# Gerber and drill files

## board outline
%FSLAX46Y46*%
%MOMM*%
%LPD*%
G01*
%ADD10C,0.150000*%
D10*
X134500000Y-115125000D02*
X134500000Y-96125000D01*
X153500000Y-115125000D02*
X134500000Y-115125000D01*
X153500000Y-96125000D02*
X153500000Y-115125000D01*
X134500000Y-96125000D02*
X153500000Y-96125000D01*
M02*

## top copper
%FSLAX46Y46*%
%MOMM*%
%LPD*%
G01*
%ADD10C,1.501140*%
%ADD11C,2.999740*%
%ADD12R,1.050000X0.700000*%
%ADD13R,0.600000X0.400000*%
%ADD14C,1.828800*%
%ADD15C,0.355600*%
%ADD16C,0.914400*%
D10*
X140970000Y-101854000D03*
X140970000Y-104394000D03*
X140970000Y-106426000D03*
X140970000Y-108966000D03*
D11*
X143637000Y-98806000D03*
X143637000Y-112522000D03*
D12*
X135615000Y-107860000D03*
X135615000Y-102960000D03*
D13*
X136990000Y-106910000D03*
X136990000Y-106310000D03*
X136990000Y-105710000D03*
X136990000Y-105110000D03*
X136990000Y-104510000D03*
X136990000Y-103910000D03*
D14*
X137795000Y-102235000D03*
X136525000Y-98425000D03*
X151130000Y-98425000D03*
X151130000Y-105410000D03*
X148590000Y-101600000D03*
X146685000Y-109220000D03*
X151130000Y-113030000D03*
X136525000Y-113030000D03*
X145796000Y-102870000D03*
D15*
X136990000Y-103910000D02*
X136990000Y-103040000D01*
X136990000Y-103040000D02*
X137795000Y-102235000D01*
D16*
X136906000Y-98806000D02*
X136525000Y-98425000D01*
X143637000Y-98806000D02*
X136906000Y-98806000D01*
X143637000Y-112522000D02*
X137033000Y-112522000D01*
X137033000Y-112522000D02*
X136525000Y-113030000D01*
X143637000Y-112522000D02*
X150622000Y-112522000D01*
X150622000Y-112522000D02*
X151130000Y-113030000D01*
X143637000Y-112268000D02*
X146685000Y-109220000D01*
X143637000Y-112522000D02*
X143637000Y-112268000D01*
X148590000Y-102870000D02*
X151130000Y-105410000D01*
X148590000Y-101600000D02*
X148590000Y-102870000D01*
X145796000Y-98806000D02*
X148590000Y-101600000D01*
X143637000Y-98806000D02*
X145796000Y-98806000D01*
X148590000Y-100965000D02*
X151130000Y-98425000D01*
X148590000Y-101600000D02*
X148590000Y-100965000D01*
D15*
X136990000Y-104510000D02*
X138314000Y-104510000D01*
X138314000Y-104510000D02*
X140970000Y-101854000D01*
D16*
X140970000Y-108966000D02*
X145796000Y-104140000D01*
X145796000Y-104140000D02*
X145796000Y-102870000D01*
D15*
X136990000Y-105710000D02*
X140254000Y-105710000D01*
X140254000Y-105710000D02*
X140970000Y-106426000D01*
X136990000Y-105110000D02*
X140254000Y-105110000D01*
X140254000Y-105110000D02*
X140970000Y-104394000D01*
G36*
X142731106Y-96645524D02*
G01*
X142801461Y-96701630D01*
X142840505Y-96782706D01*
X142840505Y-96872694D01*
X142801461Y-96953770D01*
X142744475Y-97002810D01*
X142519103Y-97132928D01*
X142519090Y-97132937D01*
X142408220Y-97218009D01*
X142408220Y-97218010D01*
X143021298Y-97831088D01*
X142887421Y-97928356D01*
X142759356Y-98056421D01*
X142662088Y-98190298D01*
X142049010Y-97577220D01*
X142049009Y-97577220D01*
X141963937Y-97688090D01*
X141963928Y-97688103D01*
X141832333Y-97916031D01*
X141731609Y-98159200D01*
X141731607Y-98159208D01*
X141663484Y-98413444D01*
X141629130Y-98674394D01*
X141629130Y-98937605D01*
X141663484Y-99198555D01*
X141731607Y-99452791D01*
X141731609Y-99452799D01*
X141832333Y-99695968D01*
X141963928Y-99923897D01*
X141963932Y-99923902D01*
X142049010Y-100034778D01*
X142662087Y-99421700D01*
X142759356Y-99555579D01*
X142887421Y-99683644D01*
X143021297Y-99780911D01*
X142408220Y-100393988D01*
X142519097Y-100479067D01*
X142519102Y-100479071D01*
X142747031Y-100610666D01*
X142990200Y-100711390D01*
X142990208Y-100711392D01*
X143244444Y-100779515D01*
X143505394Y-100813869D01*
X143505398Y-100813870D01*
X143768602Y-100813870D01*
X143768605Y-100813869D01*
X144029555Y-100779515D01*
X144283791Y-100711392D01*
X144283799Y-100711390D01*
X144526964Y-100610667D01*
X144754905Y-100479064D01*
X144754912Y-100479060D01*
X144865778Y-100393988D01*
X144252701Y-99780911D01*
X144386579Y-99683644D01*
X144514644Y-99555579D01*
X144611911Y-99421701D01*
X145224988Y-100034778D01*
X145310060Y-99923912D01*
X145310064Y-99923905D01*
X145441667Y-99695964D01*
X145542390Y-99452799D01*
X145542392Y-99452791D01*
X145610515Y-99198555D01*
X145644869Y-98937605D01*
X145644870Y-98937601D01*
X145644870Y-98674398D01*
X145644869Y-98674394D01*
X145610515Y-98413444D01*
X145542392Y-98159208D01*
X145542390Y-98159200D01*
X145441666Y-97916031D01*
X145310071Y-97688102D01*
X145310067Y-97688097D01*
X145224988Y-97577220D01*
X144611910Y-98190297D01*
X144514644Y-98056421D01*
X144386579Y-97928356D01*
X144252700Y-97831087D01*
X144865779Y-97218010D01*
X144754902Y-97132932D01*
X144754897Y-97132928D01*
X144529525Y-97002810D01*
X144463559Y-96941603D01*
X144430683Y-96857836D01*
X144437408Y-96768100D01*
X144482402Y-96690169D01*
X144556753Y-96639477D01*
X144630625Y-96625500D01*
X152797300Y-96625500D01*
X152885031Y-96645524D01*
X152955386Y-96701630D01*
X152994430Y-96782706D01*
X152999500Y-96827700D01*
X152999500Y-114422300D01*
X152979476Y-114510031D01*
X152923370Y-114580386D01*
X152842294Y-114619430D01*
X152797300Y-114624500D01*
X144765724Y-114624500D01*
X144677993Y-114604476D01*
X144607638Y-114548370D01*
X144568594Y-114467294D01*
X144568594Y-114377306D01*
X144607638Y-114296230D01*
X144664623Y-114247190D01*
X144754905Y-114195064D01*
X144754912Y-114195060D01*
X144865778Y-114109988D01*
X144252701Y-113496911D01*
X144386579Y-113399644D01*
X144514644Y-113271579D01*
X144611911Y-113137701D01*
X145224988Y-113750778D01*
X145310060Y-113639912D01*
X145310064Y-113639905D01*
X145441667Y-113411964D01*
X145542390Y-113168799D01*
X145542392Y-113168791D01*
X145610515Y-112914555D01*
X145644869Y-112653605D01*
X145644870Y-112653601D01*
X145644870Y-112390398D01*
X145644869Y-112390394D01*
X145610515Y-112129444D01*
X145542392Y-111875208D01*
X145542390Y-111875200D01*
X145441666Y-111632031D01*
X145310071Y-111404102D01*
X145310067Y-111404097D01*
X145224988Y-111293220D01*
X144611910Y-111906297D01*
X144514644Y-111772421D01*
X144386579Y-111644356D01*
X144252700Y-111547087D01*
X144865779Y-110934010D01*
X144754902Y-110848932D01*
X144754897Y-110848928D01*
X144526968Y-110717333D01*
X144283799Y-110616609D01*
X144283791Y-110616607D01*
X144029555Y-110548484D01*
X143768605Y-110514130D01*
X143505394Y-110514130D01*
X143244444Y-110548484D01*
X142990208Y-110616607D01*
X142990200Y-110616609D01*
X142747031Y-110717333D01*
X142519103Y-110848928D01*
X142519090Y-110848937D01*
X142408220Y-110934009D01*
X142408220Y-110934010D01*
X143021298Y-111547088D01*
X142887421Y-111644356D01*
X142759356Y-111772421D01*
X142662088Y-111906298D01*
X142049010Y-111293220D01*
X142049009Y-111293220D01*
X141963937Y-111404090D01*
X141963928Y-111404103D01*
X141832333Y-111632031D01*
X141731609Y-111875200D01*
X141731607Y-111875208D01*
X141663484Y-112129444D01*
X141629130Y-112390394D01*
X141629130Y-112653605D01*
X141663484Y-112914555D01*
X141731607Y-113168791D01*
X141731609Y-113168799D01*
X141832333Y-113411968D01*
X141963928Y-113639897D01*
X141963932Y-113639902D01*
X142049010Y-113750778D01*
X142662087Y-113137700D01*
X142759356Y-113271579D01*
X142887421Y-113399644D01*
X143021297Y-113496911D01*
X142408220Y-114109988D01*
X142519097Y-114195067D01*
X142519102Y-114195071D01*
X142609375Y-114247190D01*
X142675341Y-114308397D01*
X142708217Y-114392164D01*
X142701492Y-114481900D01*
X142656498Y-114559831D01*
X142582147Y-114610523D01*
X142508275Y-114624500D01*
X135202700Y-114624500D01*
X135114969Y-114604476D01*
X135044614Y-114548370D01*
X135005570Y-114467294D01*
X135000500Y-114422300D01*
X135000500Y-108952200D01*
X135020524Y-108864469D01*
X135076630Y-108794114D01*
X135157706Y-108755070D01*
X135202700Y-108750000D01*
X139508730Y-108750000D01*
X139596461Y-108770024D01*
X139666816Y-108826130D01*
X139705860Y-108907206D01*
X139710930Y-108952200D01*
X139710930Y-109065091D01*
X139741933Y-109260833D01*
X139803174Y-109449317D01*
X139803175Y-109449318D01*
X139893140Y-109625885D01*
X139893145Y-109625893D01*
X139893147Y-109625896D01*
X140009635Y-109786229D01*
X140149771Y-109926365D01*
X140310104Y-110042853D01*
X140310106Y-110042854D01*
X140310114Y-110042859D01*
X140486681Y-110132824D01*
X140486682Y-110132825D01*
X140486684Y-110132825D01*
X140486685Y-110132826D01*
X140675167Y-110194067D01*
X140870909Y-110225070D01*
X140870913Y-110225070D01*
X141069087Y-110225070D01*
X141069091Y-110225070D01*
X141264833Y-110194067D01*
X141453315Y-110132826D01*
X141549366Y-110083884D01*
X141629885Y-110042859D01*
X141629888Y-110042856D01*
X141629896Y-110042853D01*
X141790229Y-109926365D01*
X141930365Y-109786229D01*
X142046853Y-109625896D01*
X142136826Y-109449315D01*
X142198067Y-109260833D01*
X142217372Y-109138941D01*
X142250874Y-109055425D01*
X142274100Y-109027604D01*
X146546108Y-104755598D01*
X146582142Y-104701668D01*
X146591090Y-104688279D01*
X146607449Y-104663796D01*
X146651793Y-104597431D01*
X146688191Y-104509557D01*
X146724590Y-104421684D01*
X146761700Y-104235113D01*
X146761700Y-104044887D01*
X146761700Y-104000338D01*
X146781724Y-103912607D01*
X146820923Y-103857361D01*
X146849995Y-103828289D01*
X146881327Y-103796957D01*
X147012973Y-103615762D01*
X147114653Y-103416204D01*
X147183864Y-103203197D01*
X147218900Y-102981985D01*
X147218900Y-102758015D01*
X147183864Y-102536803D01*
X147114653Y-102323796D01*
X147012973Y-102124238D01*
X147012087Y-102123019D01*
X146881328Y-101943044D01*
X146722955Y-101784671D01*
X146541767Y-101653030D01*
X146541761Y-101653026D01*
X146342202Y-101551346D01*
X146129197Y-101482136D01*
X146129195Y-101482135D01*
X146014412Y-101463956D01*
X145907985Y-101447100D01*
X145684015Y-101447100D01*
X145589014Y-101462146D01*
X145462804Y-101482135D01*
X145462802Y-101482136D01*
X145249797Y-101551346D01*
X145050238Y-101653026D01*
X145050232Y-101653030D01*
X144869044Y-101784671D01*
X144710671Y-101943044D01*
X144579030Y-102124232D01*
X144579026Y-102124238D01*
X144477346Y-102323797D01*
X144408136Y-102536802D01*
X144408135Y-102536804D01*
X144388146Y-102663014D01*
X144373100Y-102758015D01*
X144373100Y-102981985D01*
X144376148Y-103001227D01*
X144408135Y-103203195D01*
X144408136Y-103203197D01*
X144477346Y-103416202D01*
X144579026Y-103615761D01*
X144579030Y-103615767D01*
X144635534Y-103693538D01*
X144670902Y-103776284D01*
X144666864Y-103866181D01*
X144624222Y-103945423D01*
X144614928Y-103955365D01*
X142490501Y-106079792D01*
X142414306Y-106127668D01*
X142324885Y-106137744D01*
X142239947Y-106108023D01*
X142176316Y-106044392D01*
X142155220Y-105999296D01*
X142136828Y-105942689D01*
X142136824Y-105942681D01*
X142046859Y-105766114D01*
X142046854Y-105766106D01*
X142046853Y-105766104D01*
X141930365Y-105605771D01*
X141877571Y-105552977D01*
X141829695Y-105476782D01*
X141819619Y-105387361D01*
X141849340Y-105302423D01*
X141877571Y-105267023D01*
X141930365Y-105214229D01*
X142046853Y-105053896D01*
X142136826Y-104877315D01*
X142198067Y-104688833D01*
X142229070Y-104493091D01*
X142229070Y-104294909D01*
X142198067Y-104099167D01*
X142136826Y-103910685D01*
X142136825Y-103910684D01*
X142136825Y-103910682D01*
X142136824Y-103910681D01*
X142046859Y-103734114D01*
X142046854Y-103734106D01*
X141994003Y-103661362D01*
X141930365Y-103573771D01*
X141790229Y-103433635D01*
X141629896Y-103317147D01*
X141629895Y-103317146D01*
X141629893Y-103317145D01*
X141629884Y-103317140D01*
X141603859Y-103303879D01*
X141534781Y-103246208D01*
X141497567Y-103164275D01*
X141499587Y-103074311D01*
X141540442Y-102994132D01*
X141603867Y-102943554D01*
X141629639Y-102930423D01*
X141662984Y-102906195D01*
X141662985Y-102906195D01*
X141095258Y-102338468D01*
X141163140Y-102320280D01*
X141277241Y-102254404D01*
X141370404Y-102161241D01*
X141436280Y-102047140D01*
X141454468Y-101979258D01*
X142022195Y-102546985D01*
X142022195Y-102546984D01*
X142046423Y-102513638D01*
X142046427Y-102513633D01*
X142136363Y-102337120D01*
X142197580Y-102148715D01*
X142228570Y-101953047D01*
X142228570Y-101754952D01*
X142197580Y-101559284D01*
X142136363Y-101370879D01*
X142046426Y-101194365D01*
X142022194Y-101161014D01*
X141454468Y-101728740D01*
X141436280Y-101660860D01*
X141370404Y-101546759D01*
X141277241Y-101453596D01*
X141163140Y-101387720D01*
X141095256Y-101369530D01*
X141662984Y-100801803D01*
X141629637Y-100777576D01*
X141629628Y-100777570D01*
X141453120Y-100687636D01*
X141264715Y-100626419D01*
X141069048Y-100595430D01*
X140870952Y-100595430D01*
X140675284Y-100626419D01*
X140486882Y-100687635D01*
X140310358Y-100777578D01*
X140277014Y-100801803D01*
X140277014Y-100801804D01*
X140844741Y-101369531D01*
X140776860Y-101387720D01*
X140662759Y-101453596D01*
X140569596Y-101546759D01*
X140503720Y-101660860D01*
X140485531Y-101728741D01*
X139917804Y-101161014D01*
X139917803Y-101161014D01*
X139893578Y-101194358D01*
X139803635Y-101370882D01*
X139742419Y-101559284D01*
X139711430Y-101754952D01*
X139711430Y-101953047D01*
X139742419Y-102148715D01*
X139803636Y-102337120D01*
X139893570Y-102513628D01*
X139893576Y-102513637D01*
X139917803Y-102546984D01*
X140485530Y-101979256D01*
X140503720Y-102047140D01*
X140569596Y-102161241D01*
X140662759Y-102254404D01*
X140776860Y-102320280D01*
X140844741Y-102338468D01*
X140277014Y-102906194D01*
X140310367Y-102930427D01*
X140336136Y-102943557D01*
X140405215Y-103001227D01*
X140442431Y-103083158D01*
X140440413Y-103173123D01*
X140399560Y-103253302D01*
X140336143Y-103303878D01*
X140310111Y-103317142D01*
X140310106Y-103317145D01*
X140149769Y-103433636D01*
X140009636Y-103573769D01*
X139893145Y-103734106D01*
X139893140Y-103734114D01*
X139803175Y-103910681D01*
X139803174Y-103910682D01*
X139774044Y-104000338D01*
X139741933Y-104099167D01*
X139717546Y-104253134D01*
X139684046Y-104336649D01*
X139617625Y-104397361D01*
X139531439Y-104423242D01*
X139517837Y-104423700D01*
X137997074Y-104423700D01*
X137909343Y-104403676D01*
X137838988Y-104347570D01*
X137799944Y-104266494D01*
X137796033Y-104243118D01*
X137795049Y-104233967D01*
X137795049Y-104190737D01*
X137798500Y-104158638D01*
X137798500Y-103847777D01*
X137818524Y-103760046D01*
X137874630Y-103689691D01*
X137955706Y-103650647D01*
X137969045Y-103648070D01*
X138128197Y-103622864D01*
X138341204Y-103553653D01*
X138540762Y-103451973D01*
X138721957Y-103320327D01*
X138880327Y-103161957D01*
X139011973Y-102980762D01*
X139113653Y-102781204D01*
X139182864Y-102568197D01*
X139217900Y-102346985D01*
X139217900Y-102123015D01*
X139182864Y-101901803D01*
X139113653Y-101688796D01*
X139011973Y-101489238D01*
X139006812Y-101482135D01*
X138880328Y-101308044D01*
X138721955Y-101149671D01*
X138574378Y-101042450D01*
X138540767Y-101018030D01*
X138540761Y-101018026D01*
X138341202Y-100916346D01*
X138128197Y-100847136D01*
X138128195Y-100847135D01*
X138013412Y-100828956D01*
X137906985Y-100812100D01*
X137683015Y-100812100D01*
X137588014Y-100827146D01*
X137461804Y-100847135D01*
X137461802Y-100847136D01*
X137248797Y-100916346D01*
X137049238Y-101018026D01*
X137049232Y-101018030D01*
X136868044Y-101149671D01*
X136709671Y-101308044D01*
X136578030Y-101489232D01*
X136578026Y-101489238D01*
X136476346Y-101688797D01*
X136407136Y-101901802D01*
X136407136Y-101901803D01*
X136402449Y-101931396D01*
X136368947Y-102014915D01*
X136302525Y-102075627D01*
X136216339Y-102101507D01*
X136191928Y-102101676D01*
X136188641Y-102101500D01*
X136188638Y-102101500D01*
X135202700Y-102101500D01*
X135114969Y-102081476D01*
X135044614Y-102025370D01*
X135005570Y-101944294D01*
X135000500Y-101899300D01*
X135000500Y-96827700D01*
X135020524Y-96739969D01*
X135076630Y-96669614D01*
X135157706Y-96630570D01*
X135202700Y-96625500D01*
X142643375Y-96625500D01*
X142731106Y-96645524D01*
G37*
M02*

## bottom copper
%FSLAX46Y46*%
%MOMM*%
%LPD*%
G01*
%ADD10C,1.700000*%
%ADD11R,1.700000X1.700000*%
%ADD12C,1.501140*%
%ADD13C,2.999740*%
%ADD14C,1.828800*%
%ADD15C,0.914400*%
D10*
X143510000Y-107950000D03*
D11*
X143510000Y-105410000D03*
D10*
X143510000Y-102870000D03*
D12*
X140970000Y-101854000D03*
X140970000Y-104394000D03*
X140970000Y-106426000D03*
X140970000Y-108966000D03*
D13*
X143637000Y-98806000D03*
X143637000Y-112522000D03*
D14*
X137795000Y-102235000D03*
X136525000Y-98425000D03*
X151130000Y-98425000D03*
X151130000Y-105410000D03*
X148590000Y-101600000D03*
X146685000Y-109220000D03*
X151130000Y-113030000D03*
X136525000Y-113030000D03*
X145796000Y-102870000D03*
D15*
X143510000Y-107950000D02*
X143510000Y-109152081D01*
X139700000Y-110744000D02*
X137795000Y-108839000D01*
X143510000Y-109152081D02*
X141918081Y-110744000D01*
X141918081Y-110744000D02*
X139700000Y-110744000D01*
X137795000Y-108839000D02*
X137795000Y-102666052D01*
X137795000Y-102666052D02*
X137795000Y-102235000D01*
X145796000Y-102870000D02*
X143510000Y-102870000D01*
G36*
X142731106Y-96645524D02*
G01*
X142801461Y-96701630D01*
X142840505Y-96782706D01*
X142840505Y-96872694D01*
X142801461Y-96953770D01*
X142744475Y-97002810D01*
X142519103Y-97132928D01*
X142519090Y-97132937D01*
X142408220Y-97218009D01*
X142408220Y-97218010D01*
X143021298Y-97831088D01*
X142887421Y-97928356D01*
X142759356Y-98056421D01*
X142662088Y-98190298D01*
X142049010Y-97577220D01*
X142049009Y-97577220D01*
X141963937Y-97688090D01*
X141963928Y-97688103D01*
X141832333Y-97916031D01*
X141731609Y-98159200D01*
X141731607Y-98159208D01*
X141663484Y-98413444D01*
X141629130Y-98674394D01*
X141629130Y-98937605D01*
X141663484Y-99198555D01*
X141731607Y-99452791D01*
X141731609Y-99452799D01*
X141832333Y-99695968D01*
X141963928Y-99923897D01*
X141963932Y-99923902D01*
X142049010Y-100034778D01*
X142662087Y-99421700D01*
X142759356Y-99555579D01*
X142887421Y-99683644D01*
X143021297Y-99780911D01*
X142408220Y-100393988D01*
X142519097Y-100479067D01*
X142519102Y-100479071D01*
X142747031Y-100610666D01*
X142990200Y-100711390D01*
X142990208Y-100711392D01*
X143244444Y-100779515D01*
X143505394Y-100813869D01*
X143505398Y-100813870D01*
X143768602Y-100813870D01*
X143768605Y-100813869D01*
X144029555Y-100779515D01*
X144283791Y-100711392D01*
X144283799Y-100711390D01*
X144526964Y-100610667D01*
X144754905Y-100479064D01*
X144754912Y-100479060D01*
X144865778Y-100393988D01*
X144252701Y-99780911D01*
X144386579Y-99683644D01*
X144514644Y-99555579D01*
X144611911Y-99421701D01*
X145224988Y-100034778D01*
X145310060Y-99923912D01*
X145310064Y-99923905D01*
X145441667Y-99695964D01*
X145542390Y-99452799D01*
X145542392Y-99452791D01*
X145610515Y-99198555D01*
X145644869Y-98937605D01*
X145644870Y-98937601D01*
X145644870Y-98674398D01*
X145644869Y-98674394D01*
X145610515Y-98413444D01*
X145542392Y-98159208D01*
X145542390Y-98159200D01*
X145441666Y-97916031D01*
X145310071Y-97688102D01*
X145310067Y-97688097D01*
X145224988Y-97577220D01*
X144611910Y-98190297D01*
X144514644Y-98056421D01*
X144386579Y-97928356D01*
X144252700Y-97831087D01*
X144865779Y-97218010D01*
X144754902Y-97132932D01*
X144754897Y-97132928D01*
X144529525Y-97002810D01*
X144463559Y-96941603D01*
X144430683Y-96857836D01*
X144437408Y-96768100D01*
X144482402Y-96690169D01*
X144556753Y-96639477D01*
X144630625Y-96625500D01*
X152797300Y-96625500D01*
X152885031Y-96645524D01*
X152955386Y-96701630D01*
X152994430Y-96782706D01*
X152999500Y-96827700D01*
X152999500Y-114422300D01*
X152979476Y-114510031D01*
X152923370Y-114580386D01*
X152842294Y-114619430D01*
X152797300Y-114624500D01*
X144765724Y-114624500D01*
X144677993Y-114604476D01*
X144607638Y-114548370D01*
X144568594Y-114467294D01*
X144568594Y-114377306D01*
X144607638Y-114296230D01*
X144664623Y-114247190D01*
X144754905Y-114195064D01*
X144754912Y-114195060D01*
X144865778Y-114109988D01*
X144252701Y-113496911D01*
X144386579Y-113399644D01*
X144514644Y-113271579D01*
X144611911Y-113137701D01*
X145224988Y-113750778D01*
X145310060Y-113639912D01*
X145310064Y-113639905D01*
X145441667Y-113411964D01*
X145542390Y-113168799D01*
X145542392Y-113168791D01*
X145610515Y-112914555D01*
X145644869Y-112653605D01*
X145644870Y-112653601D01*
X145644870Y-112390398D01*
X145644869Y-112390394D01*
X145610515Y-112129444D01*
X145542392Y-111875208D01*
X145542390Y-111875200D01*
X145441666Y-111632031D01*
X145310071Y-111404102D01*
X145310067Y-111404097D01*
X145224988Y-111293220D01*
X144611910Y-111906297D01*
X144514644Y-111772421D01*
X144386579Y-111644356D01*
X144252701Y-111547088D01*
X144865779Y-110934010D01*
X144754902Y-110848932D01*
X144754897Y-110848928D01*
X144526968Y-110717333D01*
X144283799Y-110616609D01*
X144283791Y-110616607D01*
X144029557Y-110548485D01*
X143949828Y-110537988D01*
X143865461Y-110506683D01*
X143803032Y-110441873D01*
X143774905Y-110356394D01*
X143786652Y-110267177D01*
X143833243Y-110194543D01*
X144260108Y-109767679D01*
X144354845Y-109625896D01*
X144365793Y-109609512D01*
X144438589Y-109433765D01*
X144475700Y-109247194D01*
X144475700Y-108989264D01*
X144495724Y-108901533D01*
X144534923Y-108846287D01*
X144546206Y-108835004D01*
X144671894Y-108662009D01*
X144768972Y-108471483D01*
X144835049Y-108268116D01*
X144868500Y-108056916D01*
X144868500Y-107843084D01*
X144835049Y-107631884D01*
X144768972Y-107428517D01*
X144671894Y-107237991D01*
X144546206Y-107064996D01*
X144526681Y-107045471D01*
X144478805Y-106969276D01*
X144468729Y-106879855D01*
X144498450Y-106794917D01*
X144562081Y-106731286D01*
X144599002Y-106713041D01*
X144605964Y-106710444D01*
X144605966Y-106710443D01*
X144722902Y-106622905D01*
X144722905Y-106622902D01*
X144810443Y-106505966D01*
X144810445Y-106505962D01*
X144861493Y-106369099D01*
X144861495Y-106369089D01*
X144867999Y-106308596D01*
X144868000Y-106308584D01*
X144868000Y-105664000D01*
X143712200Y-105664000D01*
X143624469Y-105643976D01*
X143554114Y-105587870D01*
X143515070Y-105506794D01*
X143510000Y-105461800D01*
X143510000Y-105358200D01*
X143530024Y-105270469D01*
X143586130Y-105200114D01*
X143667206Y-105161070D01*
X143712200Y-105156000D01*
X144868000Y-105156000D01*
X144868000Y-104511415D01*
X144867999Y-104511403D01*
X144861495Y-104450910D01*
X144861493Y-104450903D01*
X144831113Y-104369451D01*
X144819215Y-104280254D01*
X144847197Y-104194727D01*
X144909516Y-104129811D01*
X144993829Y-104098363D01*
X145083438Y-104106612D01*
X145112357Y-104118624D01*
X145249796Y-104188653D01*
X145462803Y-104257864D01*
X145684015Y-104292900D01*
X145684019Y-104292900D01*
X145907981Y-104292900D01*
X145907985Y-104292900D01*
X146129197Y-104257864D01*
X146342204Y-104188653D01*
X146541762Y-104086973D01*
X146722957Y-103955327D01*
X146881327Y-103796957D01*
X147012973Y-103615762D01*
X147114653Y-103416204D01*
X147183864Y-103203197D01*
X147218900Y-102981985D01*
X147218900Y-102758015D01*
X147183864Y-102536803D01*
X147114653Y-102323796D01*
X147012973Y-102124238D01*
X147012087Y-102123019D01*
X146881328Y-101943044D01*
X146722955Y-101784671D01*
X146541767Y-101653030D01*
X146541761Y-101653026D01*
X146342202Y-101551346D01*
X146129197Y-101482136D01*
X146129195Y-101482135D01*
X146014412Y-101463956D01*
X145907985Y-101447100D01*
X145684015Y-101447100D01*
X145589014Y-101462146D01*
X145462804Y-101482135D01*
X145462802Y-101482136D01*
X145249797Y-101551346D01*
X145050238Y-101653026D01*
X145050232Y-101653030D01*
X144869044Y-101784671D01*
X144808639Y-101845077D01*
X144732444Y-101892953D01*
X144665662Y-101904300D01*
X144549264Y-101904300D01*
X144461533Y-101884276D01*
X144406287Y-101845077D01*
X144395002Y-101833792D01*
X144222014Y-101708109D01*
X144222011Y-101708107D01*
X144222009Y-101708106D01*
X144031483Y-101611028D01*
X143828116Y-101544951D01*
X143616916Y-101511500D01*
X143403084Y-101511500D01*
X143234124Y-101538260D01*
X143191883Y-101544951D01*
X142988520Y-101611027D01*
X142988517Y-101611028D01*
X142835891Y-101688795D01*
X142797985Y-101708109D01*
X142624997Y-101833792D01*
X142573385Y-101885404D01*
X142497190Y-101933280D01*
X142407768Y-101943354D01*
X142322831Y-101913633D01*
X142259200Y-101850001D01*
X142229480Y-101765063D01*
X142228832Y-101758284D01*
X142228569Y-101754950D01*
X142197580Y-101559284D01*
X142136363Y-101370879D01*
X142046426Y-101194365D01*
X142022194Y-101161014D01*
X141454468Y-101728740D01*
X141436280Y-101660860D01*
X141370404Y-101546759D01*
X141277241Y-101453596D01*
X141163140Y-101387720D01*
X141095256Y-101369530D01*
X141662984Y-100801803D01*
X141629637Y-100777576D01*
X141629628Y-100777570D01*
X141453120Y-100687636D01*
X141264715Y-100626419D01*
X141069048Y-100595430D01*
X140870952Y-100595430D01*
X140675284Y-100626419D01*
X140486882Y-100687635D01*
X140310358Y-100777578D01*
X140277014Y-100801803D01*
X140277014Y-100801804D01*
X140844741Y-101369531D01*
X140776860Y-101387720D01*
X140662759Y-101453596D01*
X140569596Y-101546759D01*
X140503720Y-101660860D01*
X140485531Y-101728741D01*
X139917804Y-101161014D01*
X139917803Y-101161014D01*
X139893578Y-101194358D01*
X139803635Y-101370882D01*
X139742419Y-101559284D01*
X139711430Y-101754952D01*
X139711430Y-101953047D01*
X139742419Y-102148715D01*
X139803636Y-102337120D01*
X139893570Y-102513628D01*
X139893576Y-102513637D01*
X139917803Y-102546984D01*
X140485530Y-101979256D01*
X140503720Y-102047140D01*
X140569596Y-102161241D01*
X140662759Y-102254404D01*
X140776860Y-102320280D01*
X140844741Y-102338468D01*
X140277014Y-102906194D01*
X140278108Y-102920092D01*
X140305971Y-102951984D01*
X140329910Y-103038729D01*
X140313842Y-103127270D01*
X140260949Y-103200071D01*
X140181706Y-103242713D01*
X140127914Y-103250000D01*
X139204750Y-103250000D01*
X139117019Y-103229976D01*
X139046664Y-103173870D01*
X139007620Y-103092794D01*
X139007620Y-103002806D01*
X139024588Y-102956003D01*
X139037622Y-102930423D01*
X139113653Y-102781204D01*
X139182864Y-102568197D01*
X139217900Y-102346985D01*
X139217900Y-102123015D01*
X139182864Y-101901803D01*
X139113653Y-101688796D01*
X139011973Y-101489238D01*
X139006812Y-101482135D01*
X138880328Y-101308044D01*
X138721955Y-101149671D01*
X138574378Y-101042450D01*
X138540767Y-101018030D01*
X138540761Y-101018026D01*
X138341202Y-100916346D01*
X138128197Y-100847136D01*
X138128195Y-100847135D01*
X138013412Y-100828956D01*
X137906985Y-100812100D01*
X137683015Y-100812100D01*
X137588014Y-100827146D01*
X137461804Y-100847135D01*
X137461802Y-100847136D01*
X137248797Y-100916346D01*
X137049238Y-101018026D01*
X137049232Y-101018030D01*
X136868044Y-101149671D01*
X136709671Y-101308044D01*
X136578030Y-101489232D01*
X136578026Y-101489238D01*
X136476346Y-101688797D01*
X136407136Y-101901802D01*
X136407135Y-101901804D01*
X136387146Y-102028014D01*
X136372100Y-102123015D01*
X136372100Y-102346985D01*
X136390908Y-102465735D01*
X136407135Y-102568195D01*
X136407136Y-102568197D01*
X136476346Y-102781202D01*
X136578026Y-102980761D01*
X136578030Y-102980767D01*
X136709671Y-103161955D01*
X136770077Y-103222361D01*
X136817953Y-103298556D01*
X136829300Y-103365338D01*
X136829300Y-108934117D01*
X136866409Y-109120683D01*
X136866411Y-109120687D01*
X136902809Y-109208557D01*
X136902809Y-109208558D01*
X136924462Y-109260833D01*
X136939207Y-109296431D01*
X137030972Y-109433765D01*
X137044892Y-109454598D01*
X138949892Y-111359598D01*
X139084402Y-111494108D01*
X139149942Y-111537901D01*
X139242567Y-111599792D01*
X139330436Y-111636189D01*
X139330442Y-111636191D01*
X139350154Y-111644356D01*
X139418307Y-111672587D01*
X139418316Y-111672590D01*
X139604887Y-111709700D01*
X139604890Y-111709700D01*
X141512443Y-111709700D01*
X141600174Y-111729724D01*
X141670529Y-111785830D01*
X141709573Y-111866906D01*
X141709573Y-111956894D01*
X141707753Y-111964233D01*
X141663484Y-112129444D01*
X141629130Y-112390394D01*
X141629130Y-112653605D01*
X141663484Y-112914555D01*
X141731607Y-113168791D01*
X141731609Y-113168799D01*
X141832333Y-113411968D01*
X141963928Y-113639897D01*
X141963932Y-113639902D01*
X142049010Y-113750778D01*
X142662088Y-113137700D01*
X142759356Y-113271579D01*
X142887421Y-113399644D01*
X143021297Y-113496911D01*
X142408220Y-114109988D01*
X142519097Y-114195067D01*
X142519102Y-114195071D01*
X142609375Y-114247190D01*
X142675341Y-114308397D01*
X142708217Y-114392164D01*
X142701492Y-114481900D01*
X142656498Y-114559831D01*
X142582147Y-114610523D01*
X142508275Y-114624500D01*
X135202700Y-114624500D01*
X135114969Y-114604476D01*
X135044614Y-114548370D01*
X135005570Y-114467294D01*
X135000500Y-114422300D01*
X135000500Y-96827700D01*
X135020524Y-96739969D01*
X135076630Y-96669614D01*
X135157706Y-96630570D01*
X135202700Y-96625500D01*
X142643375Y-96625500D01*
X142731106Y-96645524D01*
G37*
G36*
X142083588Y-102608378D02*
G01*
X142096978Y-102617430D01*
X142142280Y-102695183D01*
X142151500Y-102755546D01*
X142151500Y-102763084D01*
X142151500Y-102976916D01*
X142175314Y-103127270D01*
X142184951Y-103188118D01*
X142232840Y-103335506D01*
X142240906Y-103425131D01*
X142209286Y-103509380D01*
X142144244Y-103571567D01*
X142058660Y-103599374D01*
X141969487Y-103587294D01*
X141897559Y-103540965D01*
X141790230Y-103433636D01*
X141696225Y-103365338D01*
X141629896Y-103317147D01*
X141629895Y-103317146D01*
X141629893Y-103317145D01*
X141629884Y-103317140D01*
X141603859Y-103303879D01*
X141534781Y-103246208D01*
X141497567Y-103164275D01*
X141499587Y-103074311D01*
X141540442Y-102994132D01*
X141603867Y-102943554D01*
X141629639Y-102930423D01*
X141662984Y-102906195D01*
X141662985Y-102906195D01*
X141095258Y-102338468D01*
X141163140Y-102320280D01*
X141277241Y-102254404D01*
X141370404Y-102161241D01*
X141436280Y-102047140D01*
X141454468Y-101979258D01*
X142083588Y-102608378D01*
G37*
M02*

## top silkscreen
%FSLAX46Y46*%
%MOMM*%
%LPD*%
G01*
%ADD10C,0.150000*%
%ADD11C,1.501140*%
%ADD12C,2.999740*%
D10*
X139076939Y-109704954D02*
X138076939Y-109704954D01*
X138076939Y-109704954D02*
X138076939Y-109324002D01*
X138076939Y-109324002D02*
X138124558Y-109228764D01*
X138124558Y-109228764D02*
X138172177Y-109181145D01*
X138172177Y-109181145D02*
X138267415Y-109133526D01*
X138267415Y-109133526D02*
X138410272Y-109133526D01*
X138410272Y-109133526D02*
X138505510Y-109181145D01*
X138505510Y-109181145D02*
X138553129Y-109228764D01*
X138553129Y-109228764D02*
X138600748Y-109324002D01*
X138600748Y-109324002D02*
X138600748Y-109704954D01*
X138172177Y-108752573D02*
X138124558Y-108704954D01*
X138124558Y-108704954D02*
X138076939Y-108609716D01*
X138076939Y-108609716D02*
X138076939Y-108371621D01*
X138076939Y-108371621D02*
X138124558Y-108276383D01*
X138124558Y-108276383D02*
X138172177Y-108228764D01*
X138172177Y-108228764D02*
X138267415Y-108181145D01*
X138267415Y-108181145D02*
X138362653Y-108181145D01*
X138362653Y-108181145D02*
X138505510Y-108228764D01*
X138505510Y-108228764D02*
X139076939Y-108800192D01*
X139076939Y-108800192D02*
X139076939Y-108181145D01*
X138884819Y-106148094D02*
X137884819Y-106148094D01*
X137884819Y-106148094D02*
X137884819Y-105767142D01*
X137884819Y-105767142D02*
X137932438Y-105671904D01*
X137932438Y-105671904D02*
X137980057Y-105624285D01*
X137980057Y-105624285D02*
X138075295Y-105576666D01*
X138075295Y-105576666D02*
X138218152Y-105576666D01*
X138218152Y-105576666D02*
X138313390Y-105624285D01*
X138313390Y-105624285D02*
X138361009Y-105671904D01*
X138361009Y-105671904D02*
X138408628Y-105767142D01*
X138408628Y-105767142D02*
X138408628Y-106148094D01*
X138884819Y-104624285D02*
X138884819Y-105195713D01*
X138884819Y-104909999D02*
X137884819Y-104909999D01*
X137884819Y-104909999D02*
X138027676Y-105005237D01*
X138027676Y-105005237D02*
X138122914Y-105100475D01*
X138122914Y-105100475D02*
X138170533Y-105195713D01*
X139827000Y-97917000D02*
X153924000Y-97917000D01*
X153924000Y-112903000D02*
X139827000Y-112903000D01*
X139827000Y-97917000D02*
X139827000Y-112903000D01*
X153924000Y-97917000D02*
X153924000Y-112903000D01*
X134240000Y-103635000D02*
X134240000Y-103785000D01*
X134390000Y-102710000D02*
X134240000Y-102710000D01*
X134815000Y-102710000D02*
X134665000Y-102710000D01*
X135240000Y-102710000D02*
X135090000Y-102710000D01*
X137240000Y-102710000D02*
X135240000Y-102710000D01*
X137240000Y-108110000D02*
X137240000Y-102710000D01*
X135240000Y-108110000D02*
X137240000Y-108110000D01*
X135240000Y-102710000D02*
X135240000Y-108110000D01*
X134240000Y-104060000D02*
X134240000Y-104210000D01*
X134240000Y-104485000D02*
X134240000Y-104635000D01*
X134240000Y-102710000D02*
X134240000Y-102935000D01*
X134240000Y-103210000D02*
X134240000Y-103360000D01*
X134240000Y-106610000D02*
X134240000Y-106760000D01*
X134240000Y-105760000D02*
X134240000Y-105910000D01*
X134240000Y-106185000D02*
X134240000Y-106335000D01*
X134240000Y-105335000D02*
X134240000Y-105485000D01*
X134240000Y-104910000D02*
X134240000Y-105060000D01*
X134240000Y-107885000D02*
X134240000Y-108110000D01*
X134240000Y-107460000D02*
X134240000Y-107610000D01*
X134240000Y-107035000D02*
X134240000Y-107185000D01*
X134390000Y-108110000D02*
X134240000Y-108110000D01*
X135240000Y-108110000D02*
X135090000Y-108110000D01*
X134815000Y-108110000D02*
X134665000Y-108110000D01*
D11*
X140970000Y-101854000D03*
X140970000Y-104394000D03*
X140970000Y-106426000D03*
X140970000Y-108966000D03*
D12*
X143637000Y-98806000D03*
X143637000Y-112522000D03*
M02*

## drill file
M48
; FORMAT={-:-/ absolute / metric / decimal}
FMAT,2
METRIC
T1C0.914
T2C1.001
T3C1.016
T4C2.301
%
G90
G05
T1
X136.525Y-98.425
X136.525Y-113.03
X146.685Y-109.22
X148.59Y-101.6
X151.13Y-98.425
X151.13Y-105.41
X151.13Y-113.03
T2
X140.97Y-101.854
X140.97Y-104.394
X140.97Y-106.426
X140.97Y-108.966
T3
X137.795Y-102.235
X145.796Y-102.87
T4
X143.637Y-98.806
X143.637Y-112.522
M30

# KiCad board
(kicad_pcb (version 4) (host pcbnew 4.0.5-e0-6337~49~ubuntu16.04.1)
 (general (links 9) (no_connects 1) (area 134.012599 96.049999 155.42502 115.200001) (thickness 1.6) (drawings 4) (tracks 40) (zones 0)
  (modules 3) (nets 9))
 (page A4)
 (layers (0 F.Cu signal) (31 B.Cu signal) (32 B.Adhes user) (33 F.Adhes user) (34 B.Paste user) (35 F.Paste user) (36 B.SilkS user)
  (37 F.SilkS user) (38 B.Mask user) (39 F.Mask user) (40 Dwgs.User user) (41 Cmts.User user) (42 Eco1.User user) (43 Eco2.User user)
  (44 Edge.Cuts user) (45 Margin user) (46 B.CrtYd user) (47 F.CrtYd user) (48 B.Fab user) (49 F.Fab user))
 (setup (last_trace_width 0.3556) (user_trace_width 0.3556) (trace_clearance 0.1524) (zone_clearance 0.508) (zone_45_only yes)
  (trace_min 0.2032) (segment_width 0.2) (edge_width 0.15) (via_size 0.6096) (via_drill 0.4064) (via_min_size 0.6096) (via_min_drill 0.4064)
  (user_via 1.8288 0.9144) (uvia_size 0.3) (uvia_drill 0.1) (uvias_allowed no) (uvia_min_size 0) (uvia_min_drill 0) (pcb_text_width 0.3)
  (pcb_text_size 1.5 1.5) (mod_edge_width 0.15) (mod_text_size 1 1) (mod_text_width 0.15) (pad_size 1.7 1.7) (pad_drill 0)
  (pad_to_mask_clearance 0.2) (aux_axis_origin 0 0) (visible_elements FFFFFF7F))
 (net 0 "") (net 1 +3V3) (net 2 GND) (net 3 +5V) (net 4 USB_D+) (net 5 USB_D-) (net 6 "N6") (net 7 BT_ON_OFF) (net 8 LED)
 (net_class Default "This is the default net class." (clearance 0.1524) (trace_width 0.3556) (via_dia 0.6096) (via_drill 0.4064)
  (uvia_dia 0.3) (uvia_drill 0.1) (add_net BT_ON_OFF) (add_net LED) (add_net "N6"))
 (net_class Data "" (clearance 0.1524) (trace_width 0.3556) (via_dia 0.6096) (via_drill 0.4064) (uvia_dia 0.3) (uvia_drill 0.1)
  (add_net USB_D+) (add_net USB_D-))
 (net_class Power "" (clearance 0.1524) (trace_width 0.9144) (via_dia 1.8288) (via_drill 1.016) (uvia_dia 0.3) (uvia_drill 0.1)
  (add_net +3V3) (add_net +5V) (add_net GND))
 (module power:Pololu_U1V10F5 (layer B.Cu) (at 143.51 107.95)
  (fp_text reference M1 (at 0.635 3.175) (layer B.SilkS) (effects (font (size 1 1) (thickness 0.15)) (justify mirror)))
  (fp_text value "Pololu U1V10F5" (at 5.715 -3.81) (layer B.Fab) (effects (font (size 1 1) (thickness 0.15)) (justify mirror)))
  (pad 1 smd circle (at 0 0) (size 1.7 1.7) (layers B.Cu B.Paste B.Mask) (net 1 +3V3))
  (pad 2 smd rect (at 0 -2.54) (size 1.7 1.7) (layers B.Cu B.Paste B.Mask) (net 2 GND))
  (pad 3 smd circle (at 0 -5.08) (size 1.7 1.7) (layers B.Cu B.Paste B.Mask) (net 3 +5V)))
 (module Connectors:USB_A (layer F.Cu) (at 140.97212 108.96686 90)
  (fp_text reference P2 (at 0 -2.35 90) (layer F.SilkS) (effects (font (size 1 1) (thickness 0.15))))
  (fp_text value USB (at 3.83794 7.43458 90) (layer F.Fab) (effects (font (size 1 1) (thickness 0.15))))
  (fp_line (start 11.04986 -1.14512) (end 11.04986 12.95188) (layer F.SilkS) (width 0.15))
  (fp_line (start -3.93614 12.95188) (end -3.93614 -1.14512) (layer F.SilkS) (width 0.15))
  (fp_line (start 11.04986 -1.14512) (end -3.93614 -1.14512) (layer F.SilkS) (width 0.15))
  (fp_line (start 11.04986 12.95188) (end -3.93614 12.95188) (layer F.SilkS) (width 0.15))
  (pad 4 thru_hole circle (at 7.11286 -0.00212) (size 1.50114 1.50114) (drill 1.00076) (layers *.Cu *.Mask F.SilkS) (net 2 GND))
  (pad 3 thru_hole circle (at 4.57286 -0.00212) (size 1.50114 1.50114) (drill 1.00076) (layers *.Cu *.Mask F.SilkS) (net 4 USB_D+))
  (pad 2 thru_hole circle (at 2.54086 -0.00212) (size 1.50114 1.50114) (drill 1.00076) (layers *.Cu *.Mask F.SilkS) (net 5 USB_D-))
  (pad 1 thru_hole circle (at 0.00086 -0.00212) (size 1.50114 1.50114) (drill 1.00076) (layers *.Cu *.Mask F.SilkS) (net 3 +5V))
  (pad 5 thru_hole circle (at 10.16086 2.66488) (size 2.99974 2.99974) (drill 2.30124) (layers *.Cu *.Mask F.SilkS) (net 2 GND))
  (pad 5 thru_hole circle (at -3.55514 2.66488) (size 2.99974 2.99974) (drill 2.30124) (layers *.Cu *.Mask F.SilkS) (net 2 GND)))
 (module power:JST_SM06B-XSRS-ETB (layer F.Cu) (at 135.89 105.41 270)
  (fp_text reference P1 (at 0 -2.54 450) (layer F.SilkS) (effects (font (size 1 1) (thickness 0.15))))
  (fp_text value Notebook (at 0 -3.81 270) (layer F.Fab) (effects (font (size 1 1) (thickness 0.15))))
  (fp_line (start -1.775 1.65) (end -1.625 1.65) (layer F.SilkS) (width 0.15))
  (fp_line (start -2.7 1.5) (end -2.7 1.65) (layer F.SilkS) (width 0.15))
  (fp_line (start -2.7 1.075) (end -2.7 1.225) (layer F.SilkS) (width 0.15))
  (fp_line (start -2.7 0.65) (end -2.7 0.8) (layer F.SilkS) (width 0.15))
  (fp_line (start -2.7 -1.35) (end -2.7 0.65) (layer F.SilkS) (width 0.15))
  (fp_line (start 2.7 -1.35) (end -2.7 -1.35) (layer F.SilkS) (width 0.15))
  (fp_line (start 2.7 0.65) (end 2.7 -1.35) (layer F.SilkS) (width 0.15))
  (fp_line (start -2.7 0.65) (end 2.7 0.65) (layer F.SilkS) (width 0.15))
  (fp_line (start -1.35 1.65) (end -1.2 1.65) (layer F.SilkS) (width 0.15))
  (fp_line (start -0.925 1.65) (end -0.775 1.65) (layer F.SilkS) (width 0.15))
  (fp_line (start -2.7 1.65) (end -2.475 1.65) (layer F.SilkS) (width 0.15))
  (fp_line (start -2.2 1.65) (end -2.05 1.65) (layer F.SilkS) (width 0.15))
  (fp_line (start 1.2 1.65) (end 1.35 1.65) (layer F.SilkS) (width 0.15))
  (fp_line (start 0.35 1.65) (end 0.5 1.65) (layer F.SilkS) (width 0.15))
  (fp_line (start 0.775 1.65) (end 0.925 1.65) (layer F.SilkS) (width 0.15))
  (fp_line (start -0.075 1.65) (end 0.075 1.65) (layer F.SilkS) (width 0.15))
  (fp_line (start -0.5 1.65) (end -0.35 1.65) (layer F.SilkS) (width 0.15))
  (fp_line (start 2.475 1.65) (end 2.7 1.65) (layer F.SilkS) (width 0.15))
  (fp_line (start 2.05 1.65) (end 2.2 1.65) (layer F.SilkS) (width 0.15))
  (fp_line (start 1.625 1.65) (end 1.775 1.65) (layer F.SilkS) (width 0.15))
  (fp_line (start 2.7 1.5) (end 2.7 1.65) (layer F.SilkS) (width 0.15))
  (fp_line (start 2.7 0.65) (end 2.7 0.8) (layer F.SilkS) (width 0.15))
  (fp_line (start 2.7 1.075) (end 2.7 1.225) (layer F.SilkS) (width 0.15))
  (pad 7 smd rect (at 2.45 0.275 270) (size 0.7 1.05) (layers F.Cu F.Paste F.Mask) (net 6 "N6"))
  (pad 7 smd rect (at -2.45 0.275 270) (size 0.7 1.05) (layers F.Cu F.Paste F.Mask) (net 6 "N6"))
  (pad 6 smd rect (at 1.5 -1.1 270) (size 0.4 0.6) (layers F.Cu F.Paste F.Mask) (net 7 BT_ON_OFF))
  (pad 5 smd rect (at 0.9 -1.1 270) (size 0.4 0.6) (layers F.Cu F.Paste F.Mask) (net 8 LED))
  (pad 4 smd rect (at 0.3 -1.1 270) (size 0.4 0.6) (layers F.Cu F.Paste F.Mask) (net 5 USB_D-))
  (pad 3 smd rect (at -0.3 -1.1 270) (size 0.4 0.6) (layers F.Cu F.Paste F.Mask) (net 4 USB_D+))
  (pad 2 smd rect (at -0.9 -1.1 270) (size 0.4 0.6) (layers F.Cu F.Paste F.Mask) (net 2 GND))
  (pad 1 smd rect (at -1.5 -1.1 270) (size 0.4 0.6) (layers F.Cu F.Paste F.Mask) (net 1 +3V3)))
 (gr_line (start 134.5 115.125) (end 134.5 96.125) (layer Edge.Cuts) (width 0.15))
 (gr_line (start 153.5 115.125) (end 134.5 115.125) (layer Edge.Cuts) (width 0.15))
 (gr_line (start 153.5 96.125) (end 153.5 115.125) (layer Edge.Cuts) (width 0.15))
 (gr_line (start 134.5 96.125) (end 153.5 96.125) (layer Edge.Cuts) (width 0.15))
 (segment (start 143.51 107.95) (end 143.51 109.152081) (width 0.9144) (layer B.Cu) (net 1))
 (segment (start 139.7 110.744) (end 137.795 108.839) (width 0.9144) (layer B.Cu) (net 1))
 (segment (start 143.51 109.152081) (end 141.918081 110.744) (width 0.9144) (layer B.Cu) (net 1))
 (segment (start 141.918081 110.744) (end 139.7 110.744) (width 0.9144) (layer B.Cu) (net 1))
 (segment (start 137.795 108.839) (end 137.795 102.666052) (width 0.9144) (layer B.Cu) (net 1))
 (segment (start 137.795 102.666052) (end 137.795 102.235) (width 0.9144) (layer B.Cu) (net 1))
 (segment (start 136.99 103.91) (end 136.99 103.04) (width 0.3556) (layer F.Cu) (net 1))
 (segment (start 136.99 103.04) (end 137.795 102.235) (width 0.3556) (layer F.Cu) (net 1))
 (via (at 137.795 102.235) (size 1.8288) (drill 1.016) (layers F.Cu B.Cu) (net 1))
 (via (at 136.525 98.425) (size 1.8288) (drill 0.9144) (layers F.Cu B.Cu) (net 2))
 (segment (start 136.906 98.806) (end 136.525 98.425) (width 0.9144) (layer F.Cu) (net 2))
 (segment (start 143.637 98.806) (end 136.906 98.806) (width 0.9144) (layer F.Cu) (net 2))
 (via (at 151.13 98.425) (size 1.8288) (drill 0.9144) (layers F.Cu B.Cu) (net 2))
 (via (at 151.13 105.41) (size 1.8288) (drill 0.9144) (layers F.Cu B.Cu) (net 2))
 (via (at 148.59 101.6) (size 1.8288) (drill 0.9144) (layers F.Cu B.Cu) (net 2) (status 1000000))
 (via (at 146.685 109.22) (size 1.8288) (drill 0.9144) (layers F.Cu B.Cu) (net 2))
 (via (at 151.13 113.03) (size 1.8288) (drill 0.9144) (layers F.Cu B.Cu) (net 2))
 (via (at 136.525 113.03) (size 1.8288) (drill 0.9144) (layers F.Cu B.Cu) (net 2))
 (segment (start 143.637 112.522) (end 137.033 112.522) (width 0.9144) (layer F.Cu) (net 2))
 (segment (start 137.033 112.522) (end 136.525 113.03) (width 0.9144) (layer F.Cu) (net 2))
 (segment (start 143.637 112.522) (end 150.622 112.522) (width 0.9144) (layer F.Cu) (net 2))
 (segment (start 150.622 112.522) (end 151.13 113.03) (width 0.9144) (layer F.Cu) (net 2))
 (segment (start 143.637 112.268) (end 146.685 109.22) (width 0.9144) (layer F.Cu) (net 2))
 (segment (start 143.637 112.522) (end 143.637 112.268) (width 0.9144) (layer F.Cu) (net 2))
 (segment (start 148.59 102.87) (end 151.13 105.41) (width 0.9144) (layer F.Cu) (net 2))
 (segment (start 148.59 101.6) (end 148.59 102.87) (width 0.9144) (layer F.Cu) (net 2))
 (segment (start 145.796 98.806) (end 148.59 101.6) (width 0.9144) (layer F.Cu) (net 2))
 (segment (start 143.637 98.806) (end 145.796 98.806) (width 0.9144) (layer F.Cu) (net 2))
 (segment (start 148.59 100.965) (end 151.13 98.425) (width 0.9144) (layer F.Cu) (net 2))
 (segment (start 148.59 101.6) (end 148.59 100.965) (width 0.9144) (layer F.Cu) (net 2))
 (segment (start 136.99 104.51) (end 138.314 104.51) (width 0.3556) (layer F.Cu) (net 2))
 (segment (start 138.314 104.51) (end 140.97 101.854) (width 0.3556) (layer F.Cu) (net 2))
 (segment (start 145.796 102.87) (end 143.51 102.87) (width 0.9144) (layer B.Cu) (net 3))
 (segment (start 140.97 108.966) (end 145.796 104.14) (width 0.9144) (layer F.Cu) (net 3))
 (segment (start 145.796 104.14) (end 145.796 102.87) (width 0.9144) (layer F.Cu) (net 3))
 (via (at 145.796 102.87) (size 1.8288) (drill 1.016) (layers F.Cu B.Cu) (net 3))
 (segment (start 136.99 105.71) (end 140.254 105.71) (width 0.3556) (layer F.Cu) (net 5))
 (segment (start 140.254 105.71) (end 140.97 106.426) (width 0.3556) (layer F.Cu) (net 5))
 (segment (start 136.99 105.11) (end 140.254 105.11) (width 0.3556) (layer F.Cu) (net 4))
 (segment (start 140.254 105.11) (end 140.97 104.394) (width 0.3556) (layer F.Cu) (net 4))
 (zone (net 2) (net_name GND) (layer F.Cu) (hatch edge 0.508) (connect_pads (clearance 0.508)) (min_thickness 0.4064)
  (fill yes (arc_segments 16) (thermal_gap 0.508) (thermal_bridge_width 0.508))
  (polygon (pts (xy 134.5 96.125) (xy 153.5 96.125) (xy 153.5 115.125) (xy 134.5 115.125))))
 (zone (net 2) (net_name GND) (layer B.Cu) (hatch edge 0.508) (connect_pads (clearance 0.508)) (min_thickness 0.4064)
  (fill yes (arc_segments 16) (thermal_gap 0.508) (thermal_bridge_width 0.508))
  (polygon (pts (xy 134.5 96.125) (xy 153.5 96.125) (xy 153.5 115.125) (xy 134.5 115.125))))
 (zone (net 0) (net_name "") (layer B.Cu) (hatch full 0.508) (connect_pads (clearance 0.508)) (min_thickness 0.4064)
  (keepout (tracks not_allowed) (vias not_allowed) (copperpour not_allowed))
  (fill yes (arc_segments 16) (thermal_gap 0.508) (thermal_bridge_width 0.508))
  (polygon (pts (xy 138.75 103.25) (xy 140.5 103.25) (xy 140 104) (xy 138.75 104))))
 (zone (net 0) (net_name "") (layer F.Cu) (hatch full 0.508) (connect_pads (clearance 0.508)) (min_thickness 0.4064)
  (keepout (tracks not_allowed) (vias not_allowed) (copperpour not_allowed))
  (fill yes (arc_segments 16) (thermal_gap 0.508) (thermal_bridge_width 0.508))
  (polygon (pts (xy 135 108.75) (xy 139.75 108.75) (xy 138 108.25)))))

